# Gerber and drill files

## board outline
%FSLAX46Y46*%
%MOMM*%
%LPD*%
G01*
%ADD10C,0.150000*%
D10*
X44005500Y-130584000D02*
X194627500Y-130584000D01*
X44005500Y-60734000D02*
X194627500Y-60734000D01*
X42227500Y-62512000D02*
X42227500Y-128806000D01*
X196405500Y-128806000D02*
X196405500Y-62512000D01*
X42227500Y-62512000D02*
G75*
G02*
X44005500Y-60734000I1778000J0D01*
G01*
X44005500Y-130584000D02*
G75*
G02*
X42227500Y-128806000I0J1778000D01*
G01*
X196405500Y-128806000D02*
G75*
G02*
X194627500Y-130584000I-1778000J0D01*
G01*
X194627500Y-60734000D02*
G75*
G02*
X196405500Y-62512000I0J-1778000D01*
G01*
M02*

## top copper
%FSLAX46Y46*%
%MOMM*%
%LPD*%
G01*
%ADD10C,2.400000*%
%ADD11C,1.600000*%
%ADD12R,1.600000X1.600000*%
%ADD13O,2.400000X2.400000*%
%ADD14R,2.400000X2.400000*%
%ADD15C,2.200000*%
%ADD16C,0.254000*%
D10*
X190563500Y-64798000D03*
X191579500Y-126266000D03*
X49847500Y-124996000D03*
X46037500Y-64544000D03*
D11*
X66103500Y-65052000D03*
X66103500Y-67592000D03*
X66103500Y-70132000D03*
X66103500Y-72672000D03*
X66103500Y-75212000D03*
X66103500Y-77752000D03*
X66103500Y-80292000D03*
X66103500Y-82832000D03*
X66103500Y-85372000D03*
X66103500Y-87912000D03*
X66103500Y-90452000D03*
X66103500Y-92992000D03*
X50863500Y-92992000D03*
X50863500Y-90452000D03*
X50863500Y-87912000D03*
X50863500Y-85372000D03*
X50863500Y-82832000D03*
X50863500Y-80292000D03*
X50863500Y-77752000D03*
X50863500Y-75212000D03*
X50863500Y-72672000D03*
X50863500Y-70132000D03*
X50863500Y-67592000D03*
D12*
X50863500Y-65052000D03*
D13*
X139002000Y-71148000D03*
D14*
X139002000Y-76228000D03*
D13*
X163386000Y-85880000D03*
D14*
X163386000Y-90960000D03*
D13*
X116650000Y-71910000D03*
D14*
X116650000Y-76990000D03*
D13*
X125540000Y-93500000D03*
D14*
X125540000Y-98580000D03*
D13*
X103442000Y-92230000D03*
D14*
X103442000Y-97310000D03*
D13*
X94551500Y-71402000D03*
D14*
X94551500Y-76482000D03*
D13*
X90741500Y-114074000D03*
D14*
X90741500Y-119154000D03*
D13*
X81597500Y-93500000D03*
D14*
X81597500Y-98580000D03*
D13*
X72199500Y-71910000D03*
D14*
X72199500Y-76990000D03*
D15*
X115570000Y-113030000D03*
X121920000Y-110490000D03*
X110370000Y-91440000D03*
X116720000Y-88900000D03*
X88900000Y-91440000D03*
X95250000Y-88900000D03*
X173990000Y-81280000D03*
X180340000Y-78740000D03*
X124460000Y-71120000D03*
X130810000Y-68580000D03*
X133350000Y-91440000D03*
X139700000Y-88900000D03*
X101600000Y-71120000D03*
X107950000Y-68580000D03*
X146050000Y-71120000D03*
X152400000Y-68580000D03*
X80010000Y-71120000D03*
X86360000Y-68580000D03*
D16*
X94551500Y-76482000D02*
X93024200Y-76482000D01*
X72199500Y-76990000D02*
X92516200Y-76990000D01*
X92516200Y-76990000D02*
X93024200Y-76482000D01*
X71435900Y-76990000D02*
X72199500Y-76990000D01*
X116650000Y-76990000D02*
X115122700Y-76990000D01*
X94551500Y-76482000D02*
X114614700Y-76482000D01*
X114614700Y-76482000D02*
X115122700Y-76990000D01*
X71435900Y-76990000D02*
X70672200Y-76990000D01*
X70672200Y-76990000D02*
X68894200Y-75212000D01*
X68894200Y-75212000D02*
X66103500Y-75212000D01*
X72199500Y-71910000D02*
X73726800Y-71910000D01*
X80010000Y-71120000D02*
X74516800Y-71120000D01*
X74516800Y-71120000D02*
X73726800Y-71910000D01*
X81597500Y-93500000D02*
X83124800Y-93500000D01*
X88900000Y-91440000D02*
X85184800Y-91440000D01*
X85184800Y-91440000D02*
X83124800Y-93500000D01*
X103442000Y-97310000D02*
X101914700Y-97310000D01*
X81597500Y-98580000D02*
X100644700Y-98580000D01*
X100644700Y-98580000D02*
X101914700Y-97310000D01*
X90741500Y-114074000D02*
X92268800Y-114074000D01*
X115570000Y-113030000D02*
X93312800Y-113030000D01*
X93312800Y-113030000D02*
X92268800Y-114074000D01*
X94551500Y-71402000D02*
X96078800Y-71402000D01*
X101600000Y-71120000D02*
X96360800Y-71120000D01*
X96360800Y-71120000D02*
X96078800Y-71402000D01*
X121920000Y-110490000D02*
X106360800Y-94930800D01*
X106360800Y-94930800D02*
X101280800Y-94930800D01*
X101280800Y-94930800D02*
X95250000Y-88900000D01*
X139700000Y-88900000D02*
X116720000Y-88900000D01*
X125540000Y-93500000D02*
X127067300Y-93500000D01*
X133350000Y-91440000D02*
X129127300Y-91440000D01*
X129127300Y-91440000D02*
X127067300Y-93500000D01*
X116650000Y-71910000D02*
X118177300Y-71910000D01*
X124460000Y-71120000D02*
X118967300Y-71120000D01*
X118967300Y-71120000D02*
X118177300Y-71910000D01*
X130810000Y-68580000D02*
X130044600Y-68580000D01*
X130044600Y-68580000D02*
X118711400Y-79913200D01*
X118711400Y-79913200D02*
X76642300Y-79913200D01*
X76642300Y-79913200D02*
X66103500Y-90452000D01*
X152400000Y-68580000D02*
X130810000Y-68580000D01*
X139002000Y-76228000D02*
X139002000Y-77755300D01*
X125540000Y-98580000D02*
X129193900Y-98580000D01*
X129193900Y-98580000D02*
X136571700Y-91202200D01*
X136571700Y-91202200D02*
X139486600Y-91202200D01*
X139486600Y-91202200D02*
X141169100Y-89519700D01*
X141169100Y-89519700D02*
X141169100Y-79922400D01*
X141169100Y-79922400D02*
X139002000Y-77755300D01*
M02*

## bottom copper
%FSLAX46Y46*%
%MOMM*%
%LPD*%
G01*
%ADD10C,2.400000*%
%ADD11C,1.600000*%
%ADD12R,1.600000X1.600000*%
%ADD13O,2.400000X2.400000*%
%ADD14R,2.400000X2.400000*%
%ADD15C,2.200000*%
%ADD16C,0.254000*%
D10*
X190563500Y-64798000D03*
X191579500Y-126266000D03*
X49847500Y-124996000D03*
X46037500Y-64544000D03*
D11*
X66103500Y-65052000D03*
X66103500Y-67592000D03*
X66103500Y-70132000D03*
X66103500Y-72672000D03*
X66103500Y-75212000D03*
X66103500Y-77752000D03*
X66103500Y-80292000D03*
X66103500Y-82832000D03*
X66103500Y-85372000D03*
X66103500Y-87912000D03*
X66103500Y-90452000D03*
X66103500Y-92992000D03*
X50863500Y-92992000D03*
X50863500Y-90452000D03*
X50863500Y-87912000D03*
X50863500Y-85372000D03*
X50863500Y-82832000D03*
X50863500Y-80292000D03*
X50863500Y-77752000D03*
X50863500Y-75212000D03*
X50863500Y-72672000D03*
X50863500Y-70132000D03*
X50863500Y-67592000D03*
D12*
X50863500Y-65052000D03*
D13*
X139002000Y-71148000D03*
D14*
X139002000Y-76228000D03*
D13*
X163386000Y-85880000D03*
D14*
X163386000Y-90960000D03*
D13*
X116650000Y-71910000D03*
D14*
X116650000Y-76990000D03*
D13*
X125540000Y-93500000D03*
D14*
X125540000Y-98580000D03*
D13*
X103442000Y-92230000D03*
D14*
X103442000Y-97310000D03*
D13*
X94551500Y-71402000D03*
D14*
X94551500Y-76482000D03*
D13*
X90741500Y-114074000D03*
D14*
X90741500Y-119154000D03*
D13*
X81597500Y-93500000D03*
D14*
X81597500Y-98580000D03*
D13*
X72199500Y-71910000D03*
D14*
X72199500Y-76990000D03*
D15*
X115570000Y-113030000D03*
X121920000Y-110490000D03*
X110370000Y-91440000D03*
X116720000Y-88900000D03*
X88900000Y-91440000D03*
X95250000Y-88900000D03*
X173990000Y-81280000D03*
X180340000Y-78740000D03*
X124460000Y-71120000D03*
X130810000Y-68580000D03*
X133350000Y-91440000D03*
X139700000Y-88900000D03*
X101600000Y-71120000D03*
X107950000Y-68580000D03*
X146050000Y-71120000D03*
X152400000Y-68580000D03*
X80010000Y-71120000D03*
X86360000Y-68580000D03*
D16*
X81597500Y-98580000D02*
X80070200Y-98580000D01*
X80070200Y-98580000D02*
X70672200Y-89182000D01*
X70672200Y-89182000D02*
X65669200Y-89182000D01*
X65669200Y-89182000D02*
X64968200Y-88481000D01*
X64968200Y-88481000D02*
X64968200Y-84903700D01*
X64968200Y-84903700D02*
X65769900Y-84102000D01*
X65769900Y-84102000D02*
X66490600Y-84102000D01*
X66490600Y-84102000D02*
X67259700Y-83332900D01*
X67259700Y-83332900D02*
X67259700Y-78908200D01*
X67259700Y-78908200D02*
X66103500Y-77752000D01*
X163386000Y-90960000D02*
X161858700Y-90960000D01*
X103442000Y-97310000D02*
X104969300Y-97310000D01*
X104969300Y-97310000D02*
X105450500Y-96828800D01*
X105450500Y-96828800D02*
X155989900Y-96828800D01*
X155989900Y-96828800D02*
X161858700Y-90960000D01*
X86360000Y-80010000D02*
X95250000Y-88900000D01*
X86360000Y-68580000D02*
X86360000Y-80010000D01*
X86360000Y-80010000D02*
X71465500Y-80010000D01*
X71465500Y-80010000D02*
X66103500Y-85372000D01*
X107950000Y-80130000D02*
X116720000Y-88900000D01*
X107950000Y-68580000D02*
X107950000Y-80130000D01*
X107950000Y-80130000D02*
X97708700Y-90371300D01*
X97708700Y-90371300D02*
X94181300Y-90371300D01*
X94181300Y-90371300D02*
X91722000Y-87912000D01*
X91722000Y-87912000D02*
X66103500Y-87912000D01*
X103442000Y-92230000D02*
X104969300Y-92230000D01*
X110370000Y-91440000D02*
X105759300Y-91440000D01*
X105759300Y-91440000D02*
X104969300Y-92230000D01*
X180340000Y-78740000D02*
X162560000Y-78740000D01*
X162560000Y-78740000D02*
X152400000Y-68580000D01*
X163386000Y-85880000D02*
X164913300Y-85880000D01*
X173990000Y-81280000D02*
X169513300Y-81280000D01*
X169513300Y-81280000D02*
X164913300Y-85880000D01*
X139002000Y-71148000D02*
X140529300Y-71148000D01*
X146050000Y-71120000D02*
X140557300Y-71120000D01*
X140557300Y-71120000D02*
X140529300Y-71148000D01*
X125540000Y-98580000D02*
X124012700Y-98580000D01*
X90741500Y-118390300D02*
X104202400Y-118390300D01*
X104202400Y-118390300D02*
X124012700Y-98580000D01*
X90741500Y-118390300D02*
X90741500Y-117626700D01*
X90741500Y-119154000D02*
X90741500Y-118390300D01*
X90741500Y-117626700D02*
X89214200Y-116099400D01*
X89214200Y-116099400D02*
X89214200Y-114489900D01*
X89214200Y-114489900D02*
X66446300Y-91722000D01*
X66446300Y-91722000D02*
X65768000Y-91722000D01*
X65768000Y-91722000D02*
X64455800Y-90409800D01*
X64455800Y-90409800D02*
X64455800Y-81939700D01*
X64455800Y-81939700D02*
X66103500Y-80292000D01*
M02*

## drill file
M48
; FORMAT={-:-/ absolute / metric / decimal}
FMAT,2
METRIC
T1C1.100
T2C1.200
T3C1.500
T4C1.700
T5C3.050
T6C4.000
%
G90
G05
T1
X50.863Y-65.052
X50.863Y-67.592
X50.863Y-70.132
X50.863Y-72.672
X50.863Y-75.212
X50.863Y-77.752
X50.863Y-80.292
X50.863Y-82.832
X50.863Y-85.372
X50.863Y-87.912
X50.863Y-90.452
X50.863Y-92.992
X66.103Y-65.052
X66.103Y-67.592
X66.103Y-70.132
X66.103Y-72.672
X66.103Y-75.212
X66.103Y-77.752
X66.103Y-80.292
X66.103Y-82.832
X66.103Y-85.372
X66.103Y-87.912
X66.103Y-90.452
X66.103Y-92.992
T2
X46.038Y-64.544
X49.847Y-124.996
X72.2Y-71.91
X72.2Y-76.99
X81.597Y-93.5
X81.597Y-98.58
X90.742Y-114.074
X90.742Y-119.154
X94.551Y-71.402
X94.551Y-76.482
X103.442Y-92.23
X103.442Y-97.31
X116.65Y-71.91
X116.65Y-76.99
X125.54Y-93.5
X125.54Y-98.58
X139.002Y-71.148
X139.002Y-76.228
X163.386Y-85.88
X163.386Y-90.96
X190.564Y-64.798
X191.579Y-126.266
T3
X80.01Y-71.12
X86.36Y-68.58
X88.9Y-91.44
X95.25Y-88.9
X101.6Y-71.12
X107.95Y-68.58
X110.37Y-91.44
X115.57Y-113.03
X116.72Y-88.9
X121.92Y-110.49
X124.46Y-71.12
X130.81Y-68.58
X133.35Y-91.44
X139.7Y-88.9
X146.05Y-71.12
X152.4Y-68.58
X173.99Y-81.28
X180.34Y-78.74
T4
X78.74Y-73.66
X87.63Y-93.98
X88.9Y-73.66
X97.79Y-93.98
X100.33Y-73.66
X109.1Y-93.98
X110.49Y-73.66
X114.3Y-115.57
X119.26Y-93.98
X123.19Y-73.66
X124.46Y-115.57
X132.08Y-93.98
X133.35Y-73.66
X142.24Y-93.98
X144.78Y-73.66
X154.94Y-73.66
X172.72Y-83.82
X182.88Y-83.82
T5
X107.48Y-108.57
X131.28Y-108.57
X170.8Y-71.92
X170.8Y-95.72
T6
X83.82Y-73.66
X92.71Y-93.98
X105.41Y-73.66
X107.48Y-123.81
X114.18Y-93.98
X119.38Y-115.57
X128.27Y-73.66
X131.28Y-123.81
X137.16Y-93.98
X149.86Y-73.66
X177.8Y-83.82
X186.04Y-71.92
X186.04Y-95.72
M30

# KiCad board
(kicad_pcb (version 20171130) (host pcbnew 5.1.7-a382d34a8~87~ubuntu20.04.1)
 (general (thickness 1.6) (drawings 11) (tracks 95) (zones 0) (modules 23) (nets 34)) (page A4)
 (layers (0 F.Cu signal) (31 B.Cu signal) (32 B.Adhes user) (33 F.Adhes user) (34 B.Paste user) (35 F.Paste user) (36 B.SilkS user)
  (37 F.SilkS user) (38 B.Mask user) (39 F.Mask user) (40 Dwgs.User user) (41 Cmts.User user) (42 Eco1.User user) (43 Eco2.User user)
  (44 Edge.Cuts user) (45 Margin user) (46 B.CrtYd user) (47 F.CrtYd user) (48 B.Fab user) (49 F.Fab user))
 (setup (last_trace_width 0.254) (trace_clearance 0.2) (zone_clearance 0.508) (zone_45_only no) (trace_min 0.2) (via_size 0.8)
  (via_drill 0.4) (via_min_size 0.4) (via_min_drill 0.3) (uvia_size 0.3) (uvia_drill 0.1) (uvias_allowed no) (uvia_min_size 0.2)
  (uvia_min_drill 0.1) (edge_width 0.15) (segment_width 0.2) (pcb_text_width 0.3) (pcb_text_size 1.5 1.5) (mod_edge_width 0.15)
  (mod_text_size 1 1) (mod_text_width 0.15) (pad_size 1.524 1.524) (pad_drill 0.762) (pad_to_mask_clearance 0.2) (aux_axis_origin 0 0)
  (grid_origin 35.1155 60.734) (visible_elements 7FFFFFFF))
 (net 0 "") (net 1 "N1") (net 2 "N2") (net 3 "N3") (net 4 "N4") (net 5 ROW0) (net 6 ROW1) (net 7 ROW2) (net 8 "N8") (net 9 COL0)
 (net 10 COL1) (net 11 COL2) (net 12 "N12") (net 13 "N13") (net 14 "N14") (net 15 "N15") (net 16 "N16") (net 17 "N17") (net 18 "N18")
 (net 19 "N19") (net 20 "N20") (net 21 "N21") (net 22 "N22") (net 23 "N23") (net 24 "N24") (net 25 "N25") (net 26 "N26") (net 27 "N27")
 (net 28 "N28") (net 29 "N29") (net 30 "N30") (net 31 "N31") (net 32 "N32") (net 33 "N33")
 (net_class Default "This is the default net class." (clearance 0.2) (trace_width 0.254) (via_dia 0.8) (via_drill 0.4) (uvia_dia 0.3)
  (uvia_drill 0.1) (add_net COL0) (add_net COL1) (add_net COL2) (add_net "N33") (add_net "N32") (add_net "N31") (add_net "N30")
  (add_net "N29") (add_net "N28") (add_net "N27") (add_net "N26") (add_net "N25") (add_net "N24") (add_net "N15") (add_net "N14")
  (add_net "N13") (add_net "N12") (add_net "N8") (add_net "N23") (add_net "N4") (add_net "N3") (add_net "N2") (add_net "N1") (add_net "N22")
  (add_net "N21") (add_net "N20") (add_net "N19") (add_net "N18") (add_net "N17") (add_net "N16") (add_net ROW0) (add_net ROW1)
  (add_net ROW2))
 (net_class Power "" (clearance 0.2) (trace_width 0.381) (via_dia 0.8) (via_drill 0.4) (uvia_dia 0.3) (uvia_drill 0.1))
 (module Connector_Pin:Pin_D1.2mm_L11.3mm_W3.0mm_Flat (layer F.Cu) (at 190.5635 64.798)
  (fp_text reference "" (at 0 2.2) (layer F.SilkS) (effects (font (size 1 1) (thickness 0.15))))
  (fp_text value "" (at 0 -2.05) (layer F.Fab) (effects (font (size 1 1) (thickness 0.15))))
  (pad 1 thru_hole circle (at 0 0) (size 2.4 2.4) (drill 1.2) (layers *.Cu *.Mask)))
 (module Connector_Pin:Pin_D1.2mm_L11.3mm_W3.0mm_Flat (layer F.Cu) (at 191.5795 126.266)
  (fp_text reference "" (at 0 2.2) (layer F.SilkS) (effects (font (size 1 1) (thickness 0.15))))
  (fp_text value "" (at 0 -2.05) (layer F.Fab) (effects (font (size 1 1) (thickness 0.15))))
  (pad 1 thru_hole circle (at 0 0) (size 2.4 2.4) (drill 1.2) (layers *.Cu *.Mask)))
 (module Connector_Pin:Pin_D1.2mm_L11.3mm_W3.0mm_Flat (layer F.Cu) (at 49.8475 124.996)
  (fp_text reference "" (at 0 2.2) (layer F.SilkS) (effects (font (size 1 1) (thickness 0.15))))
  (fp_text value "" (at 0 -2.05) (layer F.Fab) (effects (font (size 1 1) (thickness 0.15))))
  (pad 1 thru_hole circle (at 0 0) (size 2.4 2.4) (drill 1.2) (layers *.Cu *.Mask)))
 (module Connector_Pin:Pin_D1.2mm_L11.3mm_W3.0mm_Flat (layer F.Cu) (at 46.0375 64.544)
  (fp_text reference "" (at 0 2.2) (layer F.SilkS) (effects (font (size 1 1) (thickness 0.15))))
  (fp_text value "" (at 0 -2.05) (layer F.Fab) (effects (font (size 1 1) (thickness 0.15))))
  (pad 1 thru_hole circle (at 0 0) (size 2.4 2.4) (drill 1.2) (layers *.Cu *.Mask)))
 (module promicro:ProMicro (layer F.Cu) (at 58.4835 79.022 270)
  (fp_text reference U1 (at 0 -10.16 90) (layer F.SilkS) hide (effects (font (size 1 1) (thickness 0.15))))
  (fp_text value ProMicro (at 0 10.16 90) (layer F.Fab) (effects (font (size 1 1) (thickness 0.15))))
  (pad 24 thru_hole circle (at -13.97 -7.62 270) (size 1.6 1.6) (drill 1.1) (layers *.Cu *.Mask F.SilkS) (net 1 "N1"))
  (pad 23 thru_hole circle (at -11.43 -7.62 270) (size 1.6 1.6) (drill 1.1) (layers *.Cu *.Mask F.SilkS) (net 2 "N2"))
  (pad 22 thru_hole circle (at -8.89 -7.62 270) (size 1.6 1.6) (drill 1.1) (layers *.Cu *.Mask F.SilkS) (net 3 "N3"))
  (pad 21 thru_hole circle (at -6.35 -7.62 270) (size 1.6 1.6) (drill 1.1) (layers *.Cu *.Mask F.SilkS) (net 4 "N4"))
  (pad 20 thru_hole circle (at -3.81 -7.62 270) (size 1.6 1.6) (drill 1.1) (layers *.Cu *.Mask F.SilkS) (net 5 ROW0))
  (pad 19 thru_hole circle (at -1.27 -7.62 270) (size 1.6 1.6) (drill 1.1) (layers *.Cu *.Mask F.SilkS) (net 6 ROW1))
  (pad 18 thru_hole circle (at 1.27 -7.62 270) (size 1.6 1.6) (drill 1.1) (layers *.Cu *.Mask F.SilkS) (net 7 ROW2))
  (pad 17 thru_hole circle (at 3.81 -7.62 270) (size 1.6 1.6) (drill 1.1) (layers *.Cu *.Mask F.SilkS) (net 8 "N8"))
  (pad 16 thru_hole circle (at 6.35 -7.62 270) (size 1.6 1.6) (drill 1.1) (layers *.Cu *.Mask F.SilkS) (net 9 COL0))
  (pad 15 thru_hole circle (at 8.89 -7.62 270) (size 1.6 1.6) (drill 1.1) (layers *.Cu *.Mask F.SilkS) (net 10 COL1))
  (pad 14 thru_hole circle (at 11.43 -7.62 270) (size 1.6 1.6) (drill 1.1) (layers *.Cu *.Mask F.SilkS) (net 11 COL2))
  (pad 13 thru_hole circle (at 13.97 -7.62 270) (size 1.6 1.6) (drill 1.1) (layers *.Cu *.Mask F.SilkS) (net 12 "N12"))
  (pad 12 thru_hole circle (at 13.97 7.62 270) (size 1.6 1.6) (drill 1.1) (layers *.Cu *.Mask F.SilkS) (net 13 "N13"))
  (pad 11 thru_hole circle (at 11.43 7.62 270) (size 1.6 1.6) (drill 1.1) (layers *.Cu *.Mask F.SilkS) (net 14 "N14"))
  (pad 10 thru_hole circle (at 8.89 7.62 270) (size 1.6 1.6) (drill 1.1) (layers *.Cu *.Mask F.SilkS) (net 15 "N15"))
  (pad 9 thru_hole circle (at 6.35 7.62 270) (size 1.6 1.6) (drill 1.1) (layers *.Cu *.Mask F.SilkS) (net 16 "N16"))
  (pad 8 thru_hole circle (at 3.81 7.62 270) (size 1.6 1.6) (drill 1.1) (layers *.Cu *.Mask F.SilkS) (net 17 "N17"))
  (pad 7 thru_hole circle (at 1.27 7.62 270) (size 1.6 1.6) (drill 1.1) (layers *.Cu *.Mask F.SilkS) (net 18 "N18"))
  (pad 6 thru_hole circle (at -1.27 7.62 270) (size 1.6 1.6) (drill 1.1) (layers *.Cu *.Mask F.SilkS) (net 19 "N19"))
  (pad 5 thru_hole circle (at -3.81 7.62 270) (size 1.6 1.6) (drill 1.1) (layers *.Cu *.Mask F.SilkS) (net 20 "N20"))
  (pad 4 thru_hole circle (at -6.35 7.62 270) (size 1.6 1.6) (drill 1.1) (layers *.Cu *.Mask F.SilkS) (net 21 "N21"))
  (pad 3 thru_hole circle (at -8.89 7.62 270) (size 1.6 1.6) (drill 1.1) (layers *.Cu *.Mask F.SilkS) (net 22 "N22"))
  (pad 2 thru_hole circle (at -11.43 7.62 270) (size 1.6 1.6) (drill 1.1) (layers *.Cu *.Mask F.SilkS) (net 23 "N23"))
  (pad 1 thru_hole rect (at -13.97 7.62 270) (size 1.6 1.6) (drill 1.1) (layers *.Cu *.Mask F.SilkS) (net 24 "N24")))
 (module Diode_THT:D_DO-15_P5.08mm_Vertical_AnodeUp (layer F.Cu) (at 139.002 76.228 90)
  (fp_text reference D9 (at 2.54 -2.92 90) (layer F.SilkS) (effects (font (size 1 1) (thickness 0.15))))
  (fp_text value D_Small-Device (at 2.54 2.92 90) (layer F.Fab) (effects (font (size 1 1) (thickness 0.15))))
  (pad 2 thru_hole oval (at 5.08 0 90) (size 2.4 2.4) (drill 1.2) (layers *.Cu *.Mask) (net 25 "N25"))
  (pad 1 thru_hole rect (at 0 0 90) (size 2.4 2.4) (drill 1.2) (layers *.Cu *.Mask) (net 7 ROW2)))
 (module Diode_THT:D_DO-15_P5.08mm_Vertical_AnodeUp (layer F.Cu) (at 163.386 90.96 90)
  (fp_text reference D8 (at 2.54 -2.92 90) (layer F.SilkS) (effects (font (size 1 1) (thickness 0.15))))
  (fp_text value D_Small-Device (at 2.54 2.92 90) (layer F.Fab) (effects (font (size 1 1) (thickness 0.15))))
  (pad 2 thru_hole oval (at 5.08 0 90) (size 2.4 2.4) (drill 1.2) (layers *.Cu *.Mask) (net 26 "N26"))
  (pad 1 thru_hole rect (at 0 0 90) (size 2.4 2.4) (drill 1.2) (layers *.Cu *.Mask) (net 6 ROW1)))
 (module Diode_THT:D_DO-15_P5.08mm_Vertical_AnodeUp (layer F.Cu) (at 116.65 76.99 90)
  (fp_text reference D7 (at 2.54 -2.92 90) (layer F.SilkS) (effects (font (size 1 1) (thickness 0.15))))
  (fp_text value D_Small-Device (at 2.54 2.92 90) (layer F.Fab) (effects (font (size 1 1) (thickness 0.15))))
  (pad 2 thru_hole oval (at 5.08 0 90) (size 2.4 2.4) (drill 1.2) (layers *.Cu *.Mask) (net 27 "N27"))
  (pad 1 thru_hole rect (at 0 0 90) (size 2.4 2.4) (drill 1.2) (layers *.Cu *.Mask) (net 5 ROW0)))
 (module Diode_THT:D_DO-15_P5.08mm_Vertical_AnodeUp (layer F.Cu) (at 125.54 98.58 90)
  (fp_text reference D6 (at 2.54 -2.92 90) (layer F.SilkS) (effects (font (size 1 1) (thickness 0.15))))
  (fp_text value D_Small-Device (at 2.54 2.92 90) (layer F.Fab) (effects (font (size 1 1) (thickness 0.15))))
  (pad 2 thru_hole oval (at 5.08 0 90) (size 2.4 2.4) (drill 1.2) (layers *.Cu *.Mask) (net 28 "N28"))
  (pad 1 thru_hole rect (at 0 0 90) (size 2.4 2.4) (drill 1.2) (layers *.Cu *.Mask) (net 7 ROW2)))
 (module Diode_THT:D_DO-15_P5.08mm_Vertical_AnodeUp (layer F.Cu) (at 103.442 97.31 90)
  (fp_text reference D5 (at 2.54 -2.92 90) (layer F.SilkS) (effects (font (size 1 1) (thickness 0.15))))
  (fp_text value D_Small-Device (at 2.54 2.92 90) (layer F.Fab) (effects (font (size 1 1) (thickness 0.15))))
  (pad 2 thru_hole oval (at 5.08 0 90) (size 2.4 2.4) (drill 1.2) (layers *.Cu *.Mask) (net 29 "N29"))
  (pad 1 thru_hole rect (at 0 0 90) (size 2.4 2.4) (drill 1.2) (layers *.Cu *.Mask) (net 6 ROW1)))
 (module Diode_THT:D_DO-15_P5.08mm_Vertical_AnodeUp (layer F.Cu) (at 94.5515 76.482 90)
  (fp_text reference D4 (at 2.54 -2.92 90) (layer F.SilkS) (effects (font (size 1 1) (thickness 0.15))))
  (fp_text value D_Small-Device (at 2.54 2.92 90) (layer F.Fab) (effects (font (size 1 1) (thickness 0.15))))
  (pad 2 thru_hole oval (at 5.08 0 90) (size 2.4 2.4) (drill 1.2) (layers *.Cu *.Mask) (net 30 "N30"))
  (pad 1 thru_hole rect (at 0 0 90) (size 2.4 2.4) (drill 1.2) (layers *.Cu *.Mask) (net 5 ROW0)))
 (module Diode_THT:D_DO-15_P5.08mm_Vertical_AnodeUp (layer F.Cu) (at 90.7415 119.154 90)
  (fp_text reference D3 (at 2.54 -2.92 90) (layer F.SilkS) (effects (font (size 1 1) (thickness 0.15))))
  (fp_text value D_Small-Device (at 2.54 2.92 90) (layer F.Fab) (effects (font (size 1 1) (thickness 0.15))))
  (pad 2 thru_hole oval (at 5.08 0 90) (size 2.4 2.4) (drill 1.2) (layers *.Cu *.Mask) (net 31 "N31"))
  (pad 1 thru_hole rect (at 0 0 90) (size 2.4 2.4) (drill 1.2) (layers *.Cu *.Mask) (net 7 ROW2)))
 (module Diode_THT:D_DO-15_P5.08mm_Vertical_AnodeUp (layer F.Cu) (at 81.5975 98.58 90)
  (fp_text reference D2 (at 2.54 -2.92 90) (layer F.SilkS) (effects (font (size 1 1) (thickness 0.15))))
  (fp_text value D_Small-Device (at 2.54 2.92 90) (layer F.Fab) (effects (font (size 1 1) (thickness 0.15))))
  (pad 2 thru_hole oval (at 5.08 0 90) (size 2.4 2.4) (drill 1.2) (layers *.Cu *.Mask) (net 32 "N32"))
  (pad 1 thru_hole rect (at 0 0 90) (size 2.4 2.4) (drill 1.2) (layers *.Cu *.Mask) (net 6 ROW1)))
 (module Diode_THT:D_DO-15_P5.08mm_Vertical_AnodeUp (layer F.Cu) (at 72.1995 76.99 90)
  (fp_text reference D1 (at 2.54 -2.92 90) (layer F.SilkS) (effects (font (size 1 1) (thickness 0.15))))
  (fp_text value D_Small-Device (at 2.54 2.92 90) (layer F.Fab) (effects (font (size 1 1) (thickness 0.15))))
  (pad 2 thru_hole oval (at 5.08 0 90) (size 2.4 2.4) (drill 1.2) (layers *.Cu *.Mask) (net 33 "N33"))
  (pad 1 thru_hole rect (at 0 0 90) (size 2.4 2.4) (drill 1.2) (layers *.Cu *.Mask) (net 5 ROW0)))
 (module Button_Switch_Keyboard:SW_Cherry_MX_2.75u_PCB (layer F.Cu) (at 121.92 110.49)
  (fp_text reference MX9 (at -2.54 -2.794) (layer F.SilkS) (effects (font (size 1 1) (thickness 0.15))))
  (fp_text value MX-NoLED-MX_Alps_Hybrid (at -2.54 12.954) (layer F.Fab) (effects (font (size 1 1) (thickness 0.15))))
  (pad "" np_thru_hole circle (at 9.36 -1.92) (size 3.05 3.05) (drill 3.05) (layers *.Cu *.Mask))
  (pad "" np_thru_hole circle (at -14.44 -1.92) (size 3.05 3.05) (drill 3.05) (layers *.Cu *.Mask))
  (pad "" np_thru_hole circle (at -14.44 13.32) (size 4 4) (drill 4) (layers *.Cu *.Mask))
  (pad "" np_thru_hole circle (at 9.36 13.32) (size 4 4) (drill 4) (layers *.Cu *.Mask))
  (pad "" np_thru_hole circle (at 2.54 5.08) (size 1.7 1.7) (drill 1.7) (layers *.Cu *.Mask))
  (pad "" np_thru_hole circle (at -7.62 5.08) (size 1.7 1.7) (drill 1.7) (layers *.Cu *.Mask))
  (pad "" np_thru_hole circle (at -2.54 5.08) (size 4 4) (drill 4) (layers *.Cu *.Mask))
  (pad 2 thru_hole circle (at -6.35 2.54) (size 2.2 2.2) (drill 1.5) (layers *.Cu *.Mask) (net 31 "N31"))
  (pad 1 thru_hole circle (at 0 0) (size 2.2 2.2) (drill 1.5) (layers *.Cu *.Mask) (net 9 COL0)))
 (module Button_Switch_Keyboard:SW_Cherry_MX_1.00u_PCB (layer F.Cu) (at 116.72 88.9)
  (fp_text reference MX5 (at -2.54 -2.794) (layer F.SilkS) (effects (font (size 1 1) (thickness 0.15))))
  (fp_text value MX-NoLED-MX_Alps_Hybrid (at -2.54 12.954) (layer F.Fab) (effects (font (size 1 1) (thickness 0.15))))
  (pad "" np_thru_hole circle (at 2.54 5.08) (size 1.7 1.7) (drill 1.7) (layers *.Cu *.Mask))
  (pad "" np_thru_hole circle (at -7.62 5.08) (size 1.7 1.7) (drill 1.7) (layers *.Cu *.Mask))
  (pad "" np_thru_hole circle (at -2.54 5.08) (size 4 4) (drill 4) (layers *.Cu *.Mask))
  (pad 2 thru_hole circle (at -6.35 2.54) (size 2.2 2.2) (drill 1.5) (layers *.Cu *.Mask) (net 29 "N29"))
  (pad 1 thru_hole circle (at 0 0) (size 2.2 2.2) (drill 1.5) (layers *.Cu *.Mask) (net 10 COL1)))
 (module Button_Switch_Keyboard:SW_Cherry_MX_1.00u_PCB (layer F.Cu) (at 95.25 88.9)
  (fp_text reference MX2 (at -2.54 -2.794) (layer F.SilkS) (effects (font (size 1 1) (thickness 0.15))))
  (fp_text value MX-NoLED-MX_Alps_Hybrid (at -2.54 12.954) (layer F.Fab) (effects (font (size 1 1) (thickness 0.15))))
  (pad "" np_thru_hole circle (at 2.54 5.08) (size 1.7 1.7) (drill 1.7) (layers *.Cu *.Mask))
  (pad "" np_thru_hole circle (at -7.62 5.08) (size 1.7 1.7) (drill 1.7) (layers *.Cu *.Mask))
  (pad "" np_thru_hole circle (at -2.54 5.08) (size 4 4) (drill 4) (layers *.Cu *.Mask))
  (pad 2 thru_hole circle (at -6.35 2.54) (size 2.2 2.2) (drill 1.5) (layers *.Cu *.Mask) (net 32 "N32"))
  (pad 1 thru_hole circle (at 0 0) (size 2.2 2.2) (drill 1.5) (layers *.Cu *.Mask) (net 9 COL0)))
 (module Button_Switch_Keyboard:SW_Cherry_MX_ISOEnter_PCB (layer F.Cu) (at 180.34 78.74)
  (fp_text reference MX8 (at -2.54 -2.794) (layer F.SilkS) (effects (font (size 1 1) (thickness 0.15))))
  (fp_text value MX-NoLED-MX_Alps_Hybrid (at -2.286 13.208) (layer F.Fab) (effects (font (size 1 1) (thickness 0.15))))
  (pad "" np_thru_hole circle (at -9.54 -6.82) (size 3.05 3.05) (drill 3.05) (layers *.Cu *.Mask))
  (pad "" np_thru_hole circle (at -9.54 16.98) (size 3.05 3.05) (drill 3.05) (layers *.Cu *.Mask))
  (pad "" np_thru_hole circle (at 5.7 16.98) (size 4 4) (drill 4) (layers *.Cu *.Mask))
  (pad "" np_thru_hole circle (at 5.7 -6.82) (size 4 4) (drill 4) (layers *.Cu *.Mask))
  (pad "" np_thru_hole circle (at 2.54 5.08) (size 1.7 1.7) (drill 1.7) (layers *.Cu *.Mask))
  (pad "" np_thru_hole circle (at -7.62 5.08) (size 1.7 1.7) (drill 1.7) (layers *.Cu *.Mask))
  (pad "" np_thru_hole circle (at -2.54 5.08) (size 4 4) (drill 4) (layers *.Cu *.Mask))
  (pad 2 thru_hole circle (at -6.35 2.54) (size 2.2 2.2) (drill 1.5) (layers *.Cu *.Mask) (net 26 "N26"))
  (pad 1 thru_hole circle (at 0 0) (size 2.2 2.2) (drill 1.5) (layers *.Cu *.Mask) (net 11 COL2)))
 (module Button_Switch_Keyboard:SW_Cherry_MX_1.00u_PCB (layer F.Cu) (at 130.81 68.58)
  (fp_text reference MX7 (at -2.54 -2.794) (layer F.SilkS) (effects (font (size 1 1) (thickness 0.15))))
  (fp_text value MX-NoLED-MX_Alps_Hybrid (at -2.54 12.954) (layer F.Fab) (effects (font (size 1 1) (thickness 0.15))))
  (pad "" np_thru_hole circle (at 2.54 5.08) (size 1.7 1.7) (drill 1.7) (layers *.Cu *.Mask))
  (pad "" np_thru_hole circle (at -7.62 5.08) (size 1.7 1.7) (drill 1.7) (layers *.Cu *.Mask))
  (pad "" np_thru_hole circle (at -2.54 5.08) (size 4 4) (drill 4) (layers *.Cu *.Mask))
  (pad 2 thru_hole circle (at -6.35 2.54) (size 2.2 2.2) (drill 1.5) (layers *.Cu *.Mask) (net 27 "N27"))
  (pad 1 thru_hole circle (at 0 0) (size 2.2 2.2) (drill 1.5) (layers *.Cu *.Mask) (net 11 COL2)))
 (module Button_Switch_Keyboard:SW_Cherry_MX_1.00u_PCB (layer F.Cu) (at 139.7 88.9)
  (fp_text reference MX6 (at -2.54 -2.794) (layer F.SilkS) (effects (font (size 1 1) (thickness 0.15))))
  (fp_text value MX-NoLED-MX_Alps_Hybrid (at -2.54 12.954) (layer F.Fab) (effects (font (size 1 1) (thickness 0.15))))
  (pad "" np_thru_hole circle (at 2.54 5.08) (size 1.7 1.7) (drill 1.7) (layers *.Cu *.Mask))
  (pad "" np_thru_hole circle (at -7.62 5.08) (size 1.7 1.7) (drill 1.7) (layers *.Cu *.Mask))
  (pad "" np_thru_hole circle (at -2.54 5.08) (size 4 4) (drill 4) (layers *.Cu *.Mask))
  (pad 2 thru_hole circle (at -6.35 2.54) (size 2.2 2.2) (drill 1.5) (layers *.Cu *.Mask) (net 28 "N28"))
  (pad 1 thru_hole circle (at 0 0) (size 2.2 2.2) (drill 1.5) (layers *.Cu *.Mask) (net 10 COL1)))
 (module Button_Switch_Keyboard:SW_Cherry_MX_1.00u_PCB (layer F.Cu) (at 107.95 68.58)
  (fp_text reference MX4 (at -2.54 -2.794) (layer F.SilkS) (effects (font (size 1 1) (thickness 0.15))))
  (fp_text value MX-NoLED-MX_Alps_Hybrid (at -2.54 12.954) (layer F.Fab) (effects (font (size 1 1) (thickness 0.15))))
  (pad "" np_thru_hole circle (at 2.54 5.08) (size 1.7 1.7) (drill 1.7) (layers *.Cu *.Mask))
  (pad "" np_thru_hole circle (at -7.62 5.08) (size 1.7 1.7) (drill 1.7) (layers *.Cu *.Mask))
  (pad "" np_thru_hole circle (at -2.54 5.08) (size 4 4) (drill 4) (layers *.Cu *.Mask))
  (pad 2 thru_hole circle (at -6.35 2.54) (size 2.2 2.2) (drill 1.5) (layers *.Cu *.Mask) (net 30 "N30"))
  (pad 1 thru_hole circle (at 0 0) (size 2.2 2.2) (drill 1.5) (layers *.Cu *.Mask) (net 10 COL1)))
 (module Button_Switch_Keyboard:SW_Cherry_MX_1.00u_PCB (layer F.Cu) (at 152.4 68.58)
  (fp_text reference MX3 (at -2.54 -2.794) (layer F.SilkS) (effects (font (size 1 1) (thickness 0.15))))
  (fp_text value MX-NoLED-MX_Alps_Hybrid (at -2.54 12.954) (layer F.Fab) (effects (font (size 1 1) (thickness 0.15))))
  (pad "" np_thru_hole circle (at 2.54 5.08) (size 1.7 1.7) (drill 1.7) (layers *.Cu *.Mask))
  (pad "" np_thru_hole circle (at -7.62 5.08) (size 1.7 1.7) (drill 1.7) (layers *.Cu *.Mask))
  (pad "" np_thru_hole circle (at -2.54 5.08) (size 4 4) (drill 4) (layers *.Cu *.Mask))
  (pad 2 thru_hole circle (at -6.35 2.54) (size 2.2 2.2) (drill 1.5) (layers *.Cu *.Mask) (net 25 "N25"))
  (pad 1 thru_hole circle (at 0 0) (size 2.2 2.2) (drill 1.5) (layers *.Cu *.Mask) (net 11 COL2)))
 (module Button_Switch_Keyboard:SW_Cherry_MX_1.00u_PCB (layer F.Cu) (at 86.36 68.58)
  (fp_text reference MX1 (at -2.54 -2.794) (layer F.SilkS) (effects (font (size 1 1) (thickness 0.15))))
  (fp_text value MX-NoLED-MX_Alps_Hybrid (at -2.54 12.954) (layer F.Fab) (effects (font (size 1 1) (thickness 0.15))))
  (pad "" np_thru_hole circle (at 2.54 5.08) (size 1.7 1.7) (drill 1.7) (layers *.Cu *.Mask))
  (pad "" np_thru_hole circle (at -7.62 5.08) (size 1.7 1.7) (drill 1.7) (layers *.Cu *.Mask))
  (pad "" np_thru_hole circle (at -2.54 5.08) (size 4 4) (drill 4) (layers *.Cu *.Mask))
  (pad 2 thru_hole circle (at -6.35 2.54) (size 2.2 2.2) (drill 1.5) (layers *.Cu *.Mask) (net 33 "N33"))
  (pad 1 thru_hole circle (at 0 0) (size 2.2 2.2) (drill 1.5) (layers *.Cu *.Mask) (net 9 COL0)))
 (gr_line (start 44.0055 130.584) (end 194.6275 130.584) (layer Edge.Cuts) (width 0.15))
 (gr_line (start 44.0055 60.734) (end 194.6275 60.734) (layer Edge.Cuts) (width 0.15))
 (gr_line (start 42.2275 62.512) (end 42.2275 128.806) (layer Edge.Cuts) (width 0.15))
 (gr_line (start 196.4055 128.806) (end 196.4055 62.512) (layer Edge.Cuts) (width 0.15))
 (gr_arc (start 44.0055 62.512) (end 44.0055 60.734) (angle -90) (layer Edge.Cuts) (width 0.15))
 (gr_arc (start 44.0055 128.806) (end 42.2275 128.806) (angle -90) (layer Edge.Cuts) (width 0.15))
 (gr_arc (start 194.6275 128.806) (end 194.6275 130.584) (angle -90) (layer Edge.Cuts) (width 0.15))
 (gr_arc (start 194.6275 62.512) (end 196.4055 62.512) (angle -90) (layer Edge.Cuts) (width 0.15))
 (segment (start 94.5515 76.482) (end 93.0242 76.482) (width 0.254) (layer F.Cu) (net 5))
 (segment (start 72.1995 76.99) (end 92.5162 76.99) (width 0.254) (layer F.Cu) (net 5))
 (segment (start 92.5162 76.99) (end 93.0242 76.482) (width 0.254) (layer F.Cu) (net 5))
 (segment (start 71.4359 76.99) (end 72.1995 76.99) (width 0.254) (layer F.Cu) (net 5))
 (segment (start 116.65 76.99) (end 115.1227 76.99) (width 0.254) (layer F.Cu) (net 5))
 (segment (start 94.5515 76.482) (end 114.6147 76.482) (width 0.254) (layer F.Cu) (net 5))
 (segment (start 114.6147 76.482) (end 115.1227 76.99) (width 0.254) (layer F.Cu) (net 5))
 (segment (start 71.4359 76.99) (end 70.6722 76.99) (width 0.254) (layer F.Cu) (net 5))
 (segment (start 70.6722 76.99) (end 68.8942 75.212) (width 0.254) (layer F.Cu) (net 5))
 (segment (start 68.8942 75.212) (end 66.1035 75.212) (width 0.254) (layer F.Cu) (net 5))
 (segment (start 72.1995 71.91) (end 73.7268 71.91) (width 0.254) (layer F.Cu) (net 33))
 (segment (start 80.01 71.12) (end 74.5168 71.12) (width 0.254) (layer F.Cu) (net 33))
 (segment (start 74.5168 71.12) (end 73.7268 71.91) (width 0.254) (layer F.Cu) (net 33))
 (segment (start 81.5975 93.5) (end 83.1248 93.5) (width 0.254) (layer F.Cu) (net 32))
 (segment (start 88.9 91.44) (end 85.1848 91.44) (width 0.254) (layer F.Cu) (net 32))
 (segment (start 85.1848 91.44) (end 83.1248 93.5) (width 0.254) (layer F.Cu) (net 32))
 (segment (start 81.5975 98.58) (end 80.0702 98.58) (width 0.254) (layer B.Cu) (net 6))
 (segment (start 80.0702 98.58) (end 70.6722 89.182) (width 0.254) (layer B.Cu) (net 6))
 (segment (start 70.6722 89.182) (end 65.6692 89.182) (width 0.254) (layer B.Cu) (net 6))
 (segment (start 65.6692 89.182) (end 64.9682 88.481) (width 0.254) (layer B.Cu) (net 6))
 (segment (start 64.9682 88.481) (end 64.9682 84.9037) (width 0.254) (layer B.Cu) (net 6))
 (segment (start 64.9682 84.9037) (end 65.7699 84.102) (width 0.254) (layer B.Cu) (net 6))
 (segment (start 65.7699 84.102) (end 66.4906 84.102) (width 0.254) (layer B.Cu) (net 6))
 (segment (start 66.4906 84.102) (end 67.2597 83.3329) (width 0.254) (layer B.Cu) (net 6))
 (segment (start 67.2597 83.3329) (end 67.2597 78.9082) (width 0.254) (layer B.Cu) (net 6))
 (segment (start 67.2597 78.9082) (end 66.1035 77.752) (width 0.254) (layer B.Cu) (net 6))
 (segment (start 103.442 97.31) (end 101.9147 97.31) (width 0.254) (layer F.Cu) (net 6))
 (segment (start 81.5975 98.58) (end 100.6447 98.58) (width 0.254) (layer F.Cu) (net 6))
 (segment (start 100.6447 98.58) (end 101.9147 97.31) (width 0.254) (layer F.Cu) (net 6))
 (segment (start 163.386 90.96) (end 161.8587 90.96) (width 0.254) (layer B.Cu) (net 6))
 (segment (start 103.442 97.31) (end 104.9693 97.31) (width 0.254) (layer B.Cu) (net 6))
 (segment (start 104.9693 97.31) (end 105.4505 96.8288) (width 0.254) (layer B.Cu) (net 6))
 (segment (start 105.4505 96.8288) (end 155.9899 96.8288) (width 0.254) (layer B.Cu) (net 6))
 (segment (start 155.9899 96.8288) (end 161.8587 90.96) (width 0.254) (layer B.Cu) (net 6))
 (segment (start 90.7415 114.074) (end 92.2688 114.074) (width 0.254) (layer F.Cu) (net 31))
 (segment (start 115.57 113.03) (end 93.3128 113.03) (width 0.254) (layer F.Cu) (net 31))
 (segment (start 93.3128 113.03) (end 92.2688 114.074) (width 0.254) (layer F.Cu) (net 31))
 (segment (start 94.5515 71.402) (end 96.0788 71.402) (width 0.254) (layer F.Cu) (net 30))
 (segment (start 101.6 71.12) (end 96.3608 71.12) (width 0.254) (layer F.Cu) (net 30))
 (segment (start 96.3608 71.12) (end 96.0788 71.402) (width 0.254) (layer F.Cu) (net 30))
 (segment (start 86.36 80.01) (end 95.25 88.9) (width 0.254) (layer B.Cu) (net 9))
 (segment (start 86.36 68.58) (end 86.36 80.01) (width 0.254) (layer B.Cu) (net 9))
 (segment (start 86.36 80.01) (end 71.4655 80.01) (width 0.254) (layer B.Cu) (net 9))
 (segment (start 71.4655 80.01) (end 66.1035 85.372) (width 0.254) (layer B.Cu) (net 9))
 (segment (start 121.92 110.49) (end 106.3608 94.9308) (width 0.254) (layer F.Cu) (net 9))
 (segment (start 106.3608 94.9308) (end 101.2808 94.9308) (width 0.254) (layer F.Cu) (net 9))
 (segment (start 101.2808 94.9308) (end 95.25 88.9) (width 0.254) (layer F.Cu) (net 9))
 (segment (start 107.95 80.13) (end 116.72 88.9) (width 0.254) (layer B.Cu) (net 10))
 (segment (start 107.95 68.58) (end 107.95 80.13) (width 0.254) (layer B.Cu) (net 10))
 (segment (start 107.95 80.13) (end 97.7087 90.3713) (width 0.254) (layer B.Cu) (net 10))
 (segment (start 97.7087 90.3713) (end 94.1813 90.3713) (width 0.254) (layer B.Cu) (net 10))
 (segment (start 94.1813 90.3713) (end 91.722 87.912) (width 0.254) (layer B.Cu) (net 10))
 (segment (start 91.722 87.912) (end 66.1035 87.912) (width 0.254) (layer B.Cu) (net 10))
 (segment (start 139.7 88.9) (end 116.72 88.9) (width 0.254) (layer F.Cu) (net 10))
 (segment (start 103.442 92.23) (end 104.9693 92.23) (width 0.254) (layer B.Cu) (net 29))
 (segment (start 110.37 91.44) (end 105.7593 91.44) (width 0.254) (layer B.Cu) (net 29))
 (segment (start 105.7593 91.44) (end 104.9693 92.23) (width 0.254) (layer B.Cu) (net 29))
 (segment (start 125.54 93.5) (end 127.0673 93.5) (width 0.254) (layer F.Cu) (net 28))
 (segment (start 133.35 91.44) (end 129.1273 91.44) (width 0.254) (layer F.Cu) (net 28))
 (segment (start 129.1273 91.44) (end 127.0673 93.5) (width 0.254) (layer F.Cu) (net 28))
 (segment (start 116.65 71.91) (end 118.1773 71.91) (width 0.254) (layer F.Cu) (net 27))
 (segment (start 124.46 71.12) (end 118.9673 71.12) (width 0.254) (layer F.Cu) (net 27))
 (segment (start 118.9673 71.12) (end 118.1773 71.91) (width 0.254) (layer F.Cu) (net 27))
 (segment (start 130.81 68.58) (end 130.0446 68.58) (width 0.254) (layer F.Cu) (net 11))
 (segment (start 130.0446 68.58) (end 118.7114 79.9132) (width 0.254) (layer F.Cu) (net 11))
 (segment (start 118.7114 79.9132) (end 76.6423 79.9132) (width 0.254) (layer F.Cu) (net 11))
 (segment (start 76.6423 79.9132) (end 66.1035 90.452) (width 0.254) (layer F.Cu) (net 11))
 (segment (start 152.4 68.58) (end 130.81 68.58) (width 0.254) (layer F.Cu) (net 11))
 (segment (start 180.34 78.74) (end 162.56 78.74) (width 0.254) (layer B.Cu) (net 11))
 (segment (start 162.56 78.74) (end 152.4 68.58) (width 0.254) (layer B.Cu) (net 11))
 (segment (start 163.386 85.88) (end 164.9133 85.88) (width 0.254) (layer B.Cu) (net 26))
 (segment (start 173.99 81.28) (end 169.5133 81.28) (width 0.254) (layer B.Cu) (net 26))
 (segment (start 169.5133 81.28) (end 164.9133 85.88) (width 0.254) (layer B.Cu) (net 26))
 (segment (start 139.002 71.148) (end 140.5293 71.148) (width 0.254) (layer B.Cu) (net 25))
 (segment (start 146.05 71.12) (end 140.5573 71.12) (width 0.254) (layer B.Cu) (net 25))
 (segment (start 140.5573 71.12) (end 140.5293 71.148) (width 0.254) (layer B.Cu) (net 25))
 (segment (start 125.54 98.58) (end 124.0127 98.58) (width 0.254) (layer B.Cu) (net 7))
 (segment (start 90.7415 118.3903) (end 104.2024 118.3903) (width 0.254) (layer B.Cu) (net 7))
 (segment (start 104.2024 118.3903) (end 124.0127 98.58) (width 0.254) (layer B.Cu) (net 7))
 (segment (start 90.7415 118.3903) (end 90.7415 117.6267) (width 0.254) (layer B.Cu) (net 7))
 (segment (start 90.7415 119.154) (end 90.7415 118.3903) (width 0.254) (layer B.Cu) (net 7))
 (segment (start 90.7415 117.6267) (end 89.2142 116.0994) (width 0.254) (layer B.Cu) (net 7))
 (segment (start 89.2142 116.0994) (end 89.2142 114.4899) (width 0.254) (layer B.Cu) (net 7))
 (segment (start 89.2142 114.4899) (end 66.4463 91.722) (width 0.254) (layer B.Cu) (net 7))
 (segment (start 66.4463 91.722) (end 65.768 91.722) (width 0.254) (layer B.Cu) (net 7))
 (segment (start 65.768 91.722) (end 64.4558 90.4098) (width 0.254) (layer B.Cu) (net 7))
 (segment (start 64.4558 90.4098) (end 64.4558 81.9397) (width 0.254) (layer B.Cu) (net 7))
 (segment (start 64.4558 81.9397) (end 66.1035 80.292) (width 0.254) (layer B.Cu) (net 7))
 (segment (start 139.002 76.228) (end 139.002 77.7553) (width 0.254) (layer F.Cu) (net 7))
 (segment (start 125.54 98.58) (end 129.1939 98.58) (width 0.254) (layer F.Cu) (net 7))
 (segment (start 129.1939 98.58) (end 136.5717 91.2022) (width 0.254) (layer F.Cu) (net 7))
 (segment (start 136.5717 91.2022) (end 139.4866 91.2022) (width 0.254) (layer F.Cu) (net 7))
 (segment (start 139.4866 91.2022) (end 141.1691 89.5197) (width 0.254) (layer F.Cu) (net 7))
 (segment (start 141.1691 89.5197) (end 141.1691 79.9224) (width 0.254) (layer F.Cu) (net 7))
 (segment (start 141.1691 79.9224) (end 139.002 77.7553) (width 0.254) (layer F.Cu) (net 7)))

